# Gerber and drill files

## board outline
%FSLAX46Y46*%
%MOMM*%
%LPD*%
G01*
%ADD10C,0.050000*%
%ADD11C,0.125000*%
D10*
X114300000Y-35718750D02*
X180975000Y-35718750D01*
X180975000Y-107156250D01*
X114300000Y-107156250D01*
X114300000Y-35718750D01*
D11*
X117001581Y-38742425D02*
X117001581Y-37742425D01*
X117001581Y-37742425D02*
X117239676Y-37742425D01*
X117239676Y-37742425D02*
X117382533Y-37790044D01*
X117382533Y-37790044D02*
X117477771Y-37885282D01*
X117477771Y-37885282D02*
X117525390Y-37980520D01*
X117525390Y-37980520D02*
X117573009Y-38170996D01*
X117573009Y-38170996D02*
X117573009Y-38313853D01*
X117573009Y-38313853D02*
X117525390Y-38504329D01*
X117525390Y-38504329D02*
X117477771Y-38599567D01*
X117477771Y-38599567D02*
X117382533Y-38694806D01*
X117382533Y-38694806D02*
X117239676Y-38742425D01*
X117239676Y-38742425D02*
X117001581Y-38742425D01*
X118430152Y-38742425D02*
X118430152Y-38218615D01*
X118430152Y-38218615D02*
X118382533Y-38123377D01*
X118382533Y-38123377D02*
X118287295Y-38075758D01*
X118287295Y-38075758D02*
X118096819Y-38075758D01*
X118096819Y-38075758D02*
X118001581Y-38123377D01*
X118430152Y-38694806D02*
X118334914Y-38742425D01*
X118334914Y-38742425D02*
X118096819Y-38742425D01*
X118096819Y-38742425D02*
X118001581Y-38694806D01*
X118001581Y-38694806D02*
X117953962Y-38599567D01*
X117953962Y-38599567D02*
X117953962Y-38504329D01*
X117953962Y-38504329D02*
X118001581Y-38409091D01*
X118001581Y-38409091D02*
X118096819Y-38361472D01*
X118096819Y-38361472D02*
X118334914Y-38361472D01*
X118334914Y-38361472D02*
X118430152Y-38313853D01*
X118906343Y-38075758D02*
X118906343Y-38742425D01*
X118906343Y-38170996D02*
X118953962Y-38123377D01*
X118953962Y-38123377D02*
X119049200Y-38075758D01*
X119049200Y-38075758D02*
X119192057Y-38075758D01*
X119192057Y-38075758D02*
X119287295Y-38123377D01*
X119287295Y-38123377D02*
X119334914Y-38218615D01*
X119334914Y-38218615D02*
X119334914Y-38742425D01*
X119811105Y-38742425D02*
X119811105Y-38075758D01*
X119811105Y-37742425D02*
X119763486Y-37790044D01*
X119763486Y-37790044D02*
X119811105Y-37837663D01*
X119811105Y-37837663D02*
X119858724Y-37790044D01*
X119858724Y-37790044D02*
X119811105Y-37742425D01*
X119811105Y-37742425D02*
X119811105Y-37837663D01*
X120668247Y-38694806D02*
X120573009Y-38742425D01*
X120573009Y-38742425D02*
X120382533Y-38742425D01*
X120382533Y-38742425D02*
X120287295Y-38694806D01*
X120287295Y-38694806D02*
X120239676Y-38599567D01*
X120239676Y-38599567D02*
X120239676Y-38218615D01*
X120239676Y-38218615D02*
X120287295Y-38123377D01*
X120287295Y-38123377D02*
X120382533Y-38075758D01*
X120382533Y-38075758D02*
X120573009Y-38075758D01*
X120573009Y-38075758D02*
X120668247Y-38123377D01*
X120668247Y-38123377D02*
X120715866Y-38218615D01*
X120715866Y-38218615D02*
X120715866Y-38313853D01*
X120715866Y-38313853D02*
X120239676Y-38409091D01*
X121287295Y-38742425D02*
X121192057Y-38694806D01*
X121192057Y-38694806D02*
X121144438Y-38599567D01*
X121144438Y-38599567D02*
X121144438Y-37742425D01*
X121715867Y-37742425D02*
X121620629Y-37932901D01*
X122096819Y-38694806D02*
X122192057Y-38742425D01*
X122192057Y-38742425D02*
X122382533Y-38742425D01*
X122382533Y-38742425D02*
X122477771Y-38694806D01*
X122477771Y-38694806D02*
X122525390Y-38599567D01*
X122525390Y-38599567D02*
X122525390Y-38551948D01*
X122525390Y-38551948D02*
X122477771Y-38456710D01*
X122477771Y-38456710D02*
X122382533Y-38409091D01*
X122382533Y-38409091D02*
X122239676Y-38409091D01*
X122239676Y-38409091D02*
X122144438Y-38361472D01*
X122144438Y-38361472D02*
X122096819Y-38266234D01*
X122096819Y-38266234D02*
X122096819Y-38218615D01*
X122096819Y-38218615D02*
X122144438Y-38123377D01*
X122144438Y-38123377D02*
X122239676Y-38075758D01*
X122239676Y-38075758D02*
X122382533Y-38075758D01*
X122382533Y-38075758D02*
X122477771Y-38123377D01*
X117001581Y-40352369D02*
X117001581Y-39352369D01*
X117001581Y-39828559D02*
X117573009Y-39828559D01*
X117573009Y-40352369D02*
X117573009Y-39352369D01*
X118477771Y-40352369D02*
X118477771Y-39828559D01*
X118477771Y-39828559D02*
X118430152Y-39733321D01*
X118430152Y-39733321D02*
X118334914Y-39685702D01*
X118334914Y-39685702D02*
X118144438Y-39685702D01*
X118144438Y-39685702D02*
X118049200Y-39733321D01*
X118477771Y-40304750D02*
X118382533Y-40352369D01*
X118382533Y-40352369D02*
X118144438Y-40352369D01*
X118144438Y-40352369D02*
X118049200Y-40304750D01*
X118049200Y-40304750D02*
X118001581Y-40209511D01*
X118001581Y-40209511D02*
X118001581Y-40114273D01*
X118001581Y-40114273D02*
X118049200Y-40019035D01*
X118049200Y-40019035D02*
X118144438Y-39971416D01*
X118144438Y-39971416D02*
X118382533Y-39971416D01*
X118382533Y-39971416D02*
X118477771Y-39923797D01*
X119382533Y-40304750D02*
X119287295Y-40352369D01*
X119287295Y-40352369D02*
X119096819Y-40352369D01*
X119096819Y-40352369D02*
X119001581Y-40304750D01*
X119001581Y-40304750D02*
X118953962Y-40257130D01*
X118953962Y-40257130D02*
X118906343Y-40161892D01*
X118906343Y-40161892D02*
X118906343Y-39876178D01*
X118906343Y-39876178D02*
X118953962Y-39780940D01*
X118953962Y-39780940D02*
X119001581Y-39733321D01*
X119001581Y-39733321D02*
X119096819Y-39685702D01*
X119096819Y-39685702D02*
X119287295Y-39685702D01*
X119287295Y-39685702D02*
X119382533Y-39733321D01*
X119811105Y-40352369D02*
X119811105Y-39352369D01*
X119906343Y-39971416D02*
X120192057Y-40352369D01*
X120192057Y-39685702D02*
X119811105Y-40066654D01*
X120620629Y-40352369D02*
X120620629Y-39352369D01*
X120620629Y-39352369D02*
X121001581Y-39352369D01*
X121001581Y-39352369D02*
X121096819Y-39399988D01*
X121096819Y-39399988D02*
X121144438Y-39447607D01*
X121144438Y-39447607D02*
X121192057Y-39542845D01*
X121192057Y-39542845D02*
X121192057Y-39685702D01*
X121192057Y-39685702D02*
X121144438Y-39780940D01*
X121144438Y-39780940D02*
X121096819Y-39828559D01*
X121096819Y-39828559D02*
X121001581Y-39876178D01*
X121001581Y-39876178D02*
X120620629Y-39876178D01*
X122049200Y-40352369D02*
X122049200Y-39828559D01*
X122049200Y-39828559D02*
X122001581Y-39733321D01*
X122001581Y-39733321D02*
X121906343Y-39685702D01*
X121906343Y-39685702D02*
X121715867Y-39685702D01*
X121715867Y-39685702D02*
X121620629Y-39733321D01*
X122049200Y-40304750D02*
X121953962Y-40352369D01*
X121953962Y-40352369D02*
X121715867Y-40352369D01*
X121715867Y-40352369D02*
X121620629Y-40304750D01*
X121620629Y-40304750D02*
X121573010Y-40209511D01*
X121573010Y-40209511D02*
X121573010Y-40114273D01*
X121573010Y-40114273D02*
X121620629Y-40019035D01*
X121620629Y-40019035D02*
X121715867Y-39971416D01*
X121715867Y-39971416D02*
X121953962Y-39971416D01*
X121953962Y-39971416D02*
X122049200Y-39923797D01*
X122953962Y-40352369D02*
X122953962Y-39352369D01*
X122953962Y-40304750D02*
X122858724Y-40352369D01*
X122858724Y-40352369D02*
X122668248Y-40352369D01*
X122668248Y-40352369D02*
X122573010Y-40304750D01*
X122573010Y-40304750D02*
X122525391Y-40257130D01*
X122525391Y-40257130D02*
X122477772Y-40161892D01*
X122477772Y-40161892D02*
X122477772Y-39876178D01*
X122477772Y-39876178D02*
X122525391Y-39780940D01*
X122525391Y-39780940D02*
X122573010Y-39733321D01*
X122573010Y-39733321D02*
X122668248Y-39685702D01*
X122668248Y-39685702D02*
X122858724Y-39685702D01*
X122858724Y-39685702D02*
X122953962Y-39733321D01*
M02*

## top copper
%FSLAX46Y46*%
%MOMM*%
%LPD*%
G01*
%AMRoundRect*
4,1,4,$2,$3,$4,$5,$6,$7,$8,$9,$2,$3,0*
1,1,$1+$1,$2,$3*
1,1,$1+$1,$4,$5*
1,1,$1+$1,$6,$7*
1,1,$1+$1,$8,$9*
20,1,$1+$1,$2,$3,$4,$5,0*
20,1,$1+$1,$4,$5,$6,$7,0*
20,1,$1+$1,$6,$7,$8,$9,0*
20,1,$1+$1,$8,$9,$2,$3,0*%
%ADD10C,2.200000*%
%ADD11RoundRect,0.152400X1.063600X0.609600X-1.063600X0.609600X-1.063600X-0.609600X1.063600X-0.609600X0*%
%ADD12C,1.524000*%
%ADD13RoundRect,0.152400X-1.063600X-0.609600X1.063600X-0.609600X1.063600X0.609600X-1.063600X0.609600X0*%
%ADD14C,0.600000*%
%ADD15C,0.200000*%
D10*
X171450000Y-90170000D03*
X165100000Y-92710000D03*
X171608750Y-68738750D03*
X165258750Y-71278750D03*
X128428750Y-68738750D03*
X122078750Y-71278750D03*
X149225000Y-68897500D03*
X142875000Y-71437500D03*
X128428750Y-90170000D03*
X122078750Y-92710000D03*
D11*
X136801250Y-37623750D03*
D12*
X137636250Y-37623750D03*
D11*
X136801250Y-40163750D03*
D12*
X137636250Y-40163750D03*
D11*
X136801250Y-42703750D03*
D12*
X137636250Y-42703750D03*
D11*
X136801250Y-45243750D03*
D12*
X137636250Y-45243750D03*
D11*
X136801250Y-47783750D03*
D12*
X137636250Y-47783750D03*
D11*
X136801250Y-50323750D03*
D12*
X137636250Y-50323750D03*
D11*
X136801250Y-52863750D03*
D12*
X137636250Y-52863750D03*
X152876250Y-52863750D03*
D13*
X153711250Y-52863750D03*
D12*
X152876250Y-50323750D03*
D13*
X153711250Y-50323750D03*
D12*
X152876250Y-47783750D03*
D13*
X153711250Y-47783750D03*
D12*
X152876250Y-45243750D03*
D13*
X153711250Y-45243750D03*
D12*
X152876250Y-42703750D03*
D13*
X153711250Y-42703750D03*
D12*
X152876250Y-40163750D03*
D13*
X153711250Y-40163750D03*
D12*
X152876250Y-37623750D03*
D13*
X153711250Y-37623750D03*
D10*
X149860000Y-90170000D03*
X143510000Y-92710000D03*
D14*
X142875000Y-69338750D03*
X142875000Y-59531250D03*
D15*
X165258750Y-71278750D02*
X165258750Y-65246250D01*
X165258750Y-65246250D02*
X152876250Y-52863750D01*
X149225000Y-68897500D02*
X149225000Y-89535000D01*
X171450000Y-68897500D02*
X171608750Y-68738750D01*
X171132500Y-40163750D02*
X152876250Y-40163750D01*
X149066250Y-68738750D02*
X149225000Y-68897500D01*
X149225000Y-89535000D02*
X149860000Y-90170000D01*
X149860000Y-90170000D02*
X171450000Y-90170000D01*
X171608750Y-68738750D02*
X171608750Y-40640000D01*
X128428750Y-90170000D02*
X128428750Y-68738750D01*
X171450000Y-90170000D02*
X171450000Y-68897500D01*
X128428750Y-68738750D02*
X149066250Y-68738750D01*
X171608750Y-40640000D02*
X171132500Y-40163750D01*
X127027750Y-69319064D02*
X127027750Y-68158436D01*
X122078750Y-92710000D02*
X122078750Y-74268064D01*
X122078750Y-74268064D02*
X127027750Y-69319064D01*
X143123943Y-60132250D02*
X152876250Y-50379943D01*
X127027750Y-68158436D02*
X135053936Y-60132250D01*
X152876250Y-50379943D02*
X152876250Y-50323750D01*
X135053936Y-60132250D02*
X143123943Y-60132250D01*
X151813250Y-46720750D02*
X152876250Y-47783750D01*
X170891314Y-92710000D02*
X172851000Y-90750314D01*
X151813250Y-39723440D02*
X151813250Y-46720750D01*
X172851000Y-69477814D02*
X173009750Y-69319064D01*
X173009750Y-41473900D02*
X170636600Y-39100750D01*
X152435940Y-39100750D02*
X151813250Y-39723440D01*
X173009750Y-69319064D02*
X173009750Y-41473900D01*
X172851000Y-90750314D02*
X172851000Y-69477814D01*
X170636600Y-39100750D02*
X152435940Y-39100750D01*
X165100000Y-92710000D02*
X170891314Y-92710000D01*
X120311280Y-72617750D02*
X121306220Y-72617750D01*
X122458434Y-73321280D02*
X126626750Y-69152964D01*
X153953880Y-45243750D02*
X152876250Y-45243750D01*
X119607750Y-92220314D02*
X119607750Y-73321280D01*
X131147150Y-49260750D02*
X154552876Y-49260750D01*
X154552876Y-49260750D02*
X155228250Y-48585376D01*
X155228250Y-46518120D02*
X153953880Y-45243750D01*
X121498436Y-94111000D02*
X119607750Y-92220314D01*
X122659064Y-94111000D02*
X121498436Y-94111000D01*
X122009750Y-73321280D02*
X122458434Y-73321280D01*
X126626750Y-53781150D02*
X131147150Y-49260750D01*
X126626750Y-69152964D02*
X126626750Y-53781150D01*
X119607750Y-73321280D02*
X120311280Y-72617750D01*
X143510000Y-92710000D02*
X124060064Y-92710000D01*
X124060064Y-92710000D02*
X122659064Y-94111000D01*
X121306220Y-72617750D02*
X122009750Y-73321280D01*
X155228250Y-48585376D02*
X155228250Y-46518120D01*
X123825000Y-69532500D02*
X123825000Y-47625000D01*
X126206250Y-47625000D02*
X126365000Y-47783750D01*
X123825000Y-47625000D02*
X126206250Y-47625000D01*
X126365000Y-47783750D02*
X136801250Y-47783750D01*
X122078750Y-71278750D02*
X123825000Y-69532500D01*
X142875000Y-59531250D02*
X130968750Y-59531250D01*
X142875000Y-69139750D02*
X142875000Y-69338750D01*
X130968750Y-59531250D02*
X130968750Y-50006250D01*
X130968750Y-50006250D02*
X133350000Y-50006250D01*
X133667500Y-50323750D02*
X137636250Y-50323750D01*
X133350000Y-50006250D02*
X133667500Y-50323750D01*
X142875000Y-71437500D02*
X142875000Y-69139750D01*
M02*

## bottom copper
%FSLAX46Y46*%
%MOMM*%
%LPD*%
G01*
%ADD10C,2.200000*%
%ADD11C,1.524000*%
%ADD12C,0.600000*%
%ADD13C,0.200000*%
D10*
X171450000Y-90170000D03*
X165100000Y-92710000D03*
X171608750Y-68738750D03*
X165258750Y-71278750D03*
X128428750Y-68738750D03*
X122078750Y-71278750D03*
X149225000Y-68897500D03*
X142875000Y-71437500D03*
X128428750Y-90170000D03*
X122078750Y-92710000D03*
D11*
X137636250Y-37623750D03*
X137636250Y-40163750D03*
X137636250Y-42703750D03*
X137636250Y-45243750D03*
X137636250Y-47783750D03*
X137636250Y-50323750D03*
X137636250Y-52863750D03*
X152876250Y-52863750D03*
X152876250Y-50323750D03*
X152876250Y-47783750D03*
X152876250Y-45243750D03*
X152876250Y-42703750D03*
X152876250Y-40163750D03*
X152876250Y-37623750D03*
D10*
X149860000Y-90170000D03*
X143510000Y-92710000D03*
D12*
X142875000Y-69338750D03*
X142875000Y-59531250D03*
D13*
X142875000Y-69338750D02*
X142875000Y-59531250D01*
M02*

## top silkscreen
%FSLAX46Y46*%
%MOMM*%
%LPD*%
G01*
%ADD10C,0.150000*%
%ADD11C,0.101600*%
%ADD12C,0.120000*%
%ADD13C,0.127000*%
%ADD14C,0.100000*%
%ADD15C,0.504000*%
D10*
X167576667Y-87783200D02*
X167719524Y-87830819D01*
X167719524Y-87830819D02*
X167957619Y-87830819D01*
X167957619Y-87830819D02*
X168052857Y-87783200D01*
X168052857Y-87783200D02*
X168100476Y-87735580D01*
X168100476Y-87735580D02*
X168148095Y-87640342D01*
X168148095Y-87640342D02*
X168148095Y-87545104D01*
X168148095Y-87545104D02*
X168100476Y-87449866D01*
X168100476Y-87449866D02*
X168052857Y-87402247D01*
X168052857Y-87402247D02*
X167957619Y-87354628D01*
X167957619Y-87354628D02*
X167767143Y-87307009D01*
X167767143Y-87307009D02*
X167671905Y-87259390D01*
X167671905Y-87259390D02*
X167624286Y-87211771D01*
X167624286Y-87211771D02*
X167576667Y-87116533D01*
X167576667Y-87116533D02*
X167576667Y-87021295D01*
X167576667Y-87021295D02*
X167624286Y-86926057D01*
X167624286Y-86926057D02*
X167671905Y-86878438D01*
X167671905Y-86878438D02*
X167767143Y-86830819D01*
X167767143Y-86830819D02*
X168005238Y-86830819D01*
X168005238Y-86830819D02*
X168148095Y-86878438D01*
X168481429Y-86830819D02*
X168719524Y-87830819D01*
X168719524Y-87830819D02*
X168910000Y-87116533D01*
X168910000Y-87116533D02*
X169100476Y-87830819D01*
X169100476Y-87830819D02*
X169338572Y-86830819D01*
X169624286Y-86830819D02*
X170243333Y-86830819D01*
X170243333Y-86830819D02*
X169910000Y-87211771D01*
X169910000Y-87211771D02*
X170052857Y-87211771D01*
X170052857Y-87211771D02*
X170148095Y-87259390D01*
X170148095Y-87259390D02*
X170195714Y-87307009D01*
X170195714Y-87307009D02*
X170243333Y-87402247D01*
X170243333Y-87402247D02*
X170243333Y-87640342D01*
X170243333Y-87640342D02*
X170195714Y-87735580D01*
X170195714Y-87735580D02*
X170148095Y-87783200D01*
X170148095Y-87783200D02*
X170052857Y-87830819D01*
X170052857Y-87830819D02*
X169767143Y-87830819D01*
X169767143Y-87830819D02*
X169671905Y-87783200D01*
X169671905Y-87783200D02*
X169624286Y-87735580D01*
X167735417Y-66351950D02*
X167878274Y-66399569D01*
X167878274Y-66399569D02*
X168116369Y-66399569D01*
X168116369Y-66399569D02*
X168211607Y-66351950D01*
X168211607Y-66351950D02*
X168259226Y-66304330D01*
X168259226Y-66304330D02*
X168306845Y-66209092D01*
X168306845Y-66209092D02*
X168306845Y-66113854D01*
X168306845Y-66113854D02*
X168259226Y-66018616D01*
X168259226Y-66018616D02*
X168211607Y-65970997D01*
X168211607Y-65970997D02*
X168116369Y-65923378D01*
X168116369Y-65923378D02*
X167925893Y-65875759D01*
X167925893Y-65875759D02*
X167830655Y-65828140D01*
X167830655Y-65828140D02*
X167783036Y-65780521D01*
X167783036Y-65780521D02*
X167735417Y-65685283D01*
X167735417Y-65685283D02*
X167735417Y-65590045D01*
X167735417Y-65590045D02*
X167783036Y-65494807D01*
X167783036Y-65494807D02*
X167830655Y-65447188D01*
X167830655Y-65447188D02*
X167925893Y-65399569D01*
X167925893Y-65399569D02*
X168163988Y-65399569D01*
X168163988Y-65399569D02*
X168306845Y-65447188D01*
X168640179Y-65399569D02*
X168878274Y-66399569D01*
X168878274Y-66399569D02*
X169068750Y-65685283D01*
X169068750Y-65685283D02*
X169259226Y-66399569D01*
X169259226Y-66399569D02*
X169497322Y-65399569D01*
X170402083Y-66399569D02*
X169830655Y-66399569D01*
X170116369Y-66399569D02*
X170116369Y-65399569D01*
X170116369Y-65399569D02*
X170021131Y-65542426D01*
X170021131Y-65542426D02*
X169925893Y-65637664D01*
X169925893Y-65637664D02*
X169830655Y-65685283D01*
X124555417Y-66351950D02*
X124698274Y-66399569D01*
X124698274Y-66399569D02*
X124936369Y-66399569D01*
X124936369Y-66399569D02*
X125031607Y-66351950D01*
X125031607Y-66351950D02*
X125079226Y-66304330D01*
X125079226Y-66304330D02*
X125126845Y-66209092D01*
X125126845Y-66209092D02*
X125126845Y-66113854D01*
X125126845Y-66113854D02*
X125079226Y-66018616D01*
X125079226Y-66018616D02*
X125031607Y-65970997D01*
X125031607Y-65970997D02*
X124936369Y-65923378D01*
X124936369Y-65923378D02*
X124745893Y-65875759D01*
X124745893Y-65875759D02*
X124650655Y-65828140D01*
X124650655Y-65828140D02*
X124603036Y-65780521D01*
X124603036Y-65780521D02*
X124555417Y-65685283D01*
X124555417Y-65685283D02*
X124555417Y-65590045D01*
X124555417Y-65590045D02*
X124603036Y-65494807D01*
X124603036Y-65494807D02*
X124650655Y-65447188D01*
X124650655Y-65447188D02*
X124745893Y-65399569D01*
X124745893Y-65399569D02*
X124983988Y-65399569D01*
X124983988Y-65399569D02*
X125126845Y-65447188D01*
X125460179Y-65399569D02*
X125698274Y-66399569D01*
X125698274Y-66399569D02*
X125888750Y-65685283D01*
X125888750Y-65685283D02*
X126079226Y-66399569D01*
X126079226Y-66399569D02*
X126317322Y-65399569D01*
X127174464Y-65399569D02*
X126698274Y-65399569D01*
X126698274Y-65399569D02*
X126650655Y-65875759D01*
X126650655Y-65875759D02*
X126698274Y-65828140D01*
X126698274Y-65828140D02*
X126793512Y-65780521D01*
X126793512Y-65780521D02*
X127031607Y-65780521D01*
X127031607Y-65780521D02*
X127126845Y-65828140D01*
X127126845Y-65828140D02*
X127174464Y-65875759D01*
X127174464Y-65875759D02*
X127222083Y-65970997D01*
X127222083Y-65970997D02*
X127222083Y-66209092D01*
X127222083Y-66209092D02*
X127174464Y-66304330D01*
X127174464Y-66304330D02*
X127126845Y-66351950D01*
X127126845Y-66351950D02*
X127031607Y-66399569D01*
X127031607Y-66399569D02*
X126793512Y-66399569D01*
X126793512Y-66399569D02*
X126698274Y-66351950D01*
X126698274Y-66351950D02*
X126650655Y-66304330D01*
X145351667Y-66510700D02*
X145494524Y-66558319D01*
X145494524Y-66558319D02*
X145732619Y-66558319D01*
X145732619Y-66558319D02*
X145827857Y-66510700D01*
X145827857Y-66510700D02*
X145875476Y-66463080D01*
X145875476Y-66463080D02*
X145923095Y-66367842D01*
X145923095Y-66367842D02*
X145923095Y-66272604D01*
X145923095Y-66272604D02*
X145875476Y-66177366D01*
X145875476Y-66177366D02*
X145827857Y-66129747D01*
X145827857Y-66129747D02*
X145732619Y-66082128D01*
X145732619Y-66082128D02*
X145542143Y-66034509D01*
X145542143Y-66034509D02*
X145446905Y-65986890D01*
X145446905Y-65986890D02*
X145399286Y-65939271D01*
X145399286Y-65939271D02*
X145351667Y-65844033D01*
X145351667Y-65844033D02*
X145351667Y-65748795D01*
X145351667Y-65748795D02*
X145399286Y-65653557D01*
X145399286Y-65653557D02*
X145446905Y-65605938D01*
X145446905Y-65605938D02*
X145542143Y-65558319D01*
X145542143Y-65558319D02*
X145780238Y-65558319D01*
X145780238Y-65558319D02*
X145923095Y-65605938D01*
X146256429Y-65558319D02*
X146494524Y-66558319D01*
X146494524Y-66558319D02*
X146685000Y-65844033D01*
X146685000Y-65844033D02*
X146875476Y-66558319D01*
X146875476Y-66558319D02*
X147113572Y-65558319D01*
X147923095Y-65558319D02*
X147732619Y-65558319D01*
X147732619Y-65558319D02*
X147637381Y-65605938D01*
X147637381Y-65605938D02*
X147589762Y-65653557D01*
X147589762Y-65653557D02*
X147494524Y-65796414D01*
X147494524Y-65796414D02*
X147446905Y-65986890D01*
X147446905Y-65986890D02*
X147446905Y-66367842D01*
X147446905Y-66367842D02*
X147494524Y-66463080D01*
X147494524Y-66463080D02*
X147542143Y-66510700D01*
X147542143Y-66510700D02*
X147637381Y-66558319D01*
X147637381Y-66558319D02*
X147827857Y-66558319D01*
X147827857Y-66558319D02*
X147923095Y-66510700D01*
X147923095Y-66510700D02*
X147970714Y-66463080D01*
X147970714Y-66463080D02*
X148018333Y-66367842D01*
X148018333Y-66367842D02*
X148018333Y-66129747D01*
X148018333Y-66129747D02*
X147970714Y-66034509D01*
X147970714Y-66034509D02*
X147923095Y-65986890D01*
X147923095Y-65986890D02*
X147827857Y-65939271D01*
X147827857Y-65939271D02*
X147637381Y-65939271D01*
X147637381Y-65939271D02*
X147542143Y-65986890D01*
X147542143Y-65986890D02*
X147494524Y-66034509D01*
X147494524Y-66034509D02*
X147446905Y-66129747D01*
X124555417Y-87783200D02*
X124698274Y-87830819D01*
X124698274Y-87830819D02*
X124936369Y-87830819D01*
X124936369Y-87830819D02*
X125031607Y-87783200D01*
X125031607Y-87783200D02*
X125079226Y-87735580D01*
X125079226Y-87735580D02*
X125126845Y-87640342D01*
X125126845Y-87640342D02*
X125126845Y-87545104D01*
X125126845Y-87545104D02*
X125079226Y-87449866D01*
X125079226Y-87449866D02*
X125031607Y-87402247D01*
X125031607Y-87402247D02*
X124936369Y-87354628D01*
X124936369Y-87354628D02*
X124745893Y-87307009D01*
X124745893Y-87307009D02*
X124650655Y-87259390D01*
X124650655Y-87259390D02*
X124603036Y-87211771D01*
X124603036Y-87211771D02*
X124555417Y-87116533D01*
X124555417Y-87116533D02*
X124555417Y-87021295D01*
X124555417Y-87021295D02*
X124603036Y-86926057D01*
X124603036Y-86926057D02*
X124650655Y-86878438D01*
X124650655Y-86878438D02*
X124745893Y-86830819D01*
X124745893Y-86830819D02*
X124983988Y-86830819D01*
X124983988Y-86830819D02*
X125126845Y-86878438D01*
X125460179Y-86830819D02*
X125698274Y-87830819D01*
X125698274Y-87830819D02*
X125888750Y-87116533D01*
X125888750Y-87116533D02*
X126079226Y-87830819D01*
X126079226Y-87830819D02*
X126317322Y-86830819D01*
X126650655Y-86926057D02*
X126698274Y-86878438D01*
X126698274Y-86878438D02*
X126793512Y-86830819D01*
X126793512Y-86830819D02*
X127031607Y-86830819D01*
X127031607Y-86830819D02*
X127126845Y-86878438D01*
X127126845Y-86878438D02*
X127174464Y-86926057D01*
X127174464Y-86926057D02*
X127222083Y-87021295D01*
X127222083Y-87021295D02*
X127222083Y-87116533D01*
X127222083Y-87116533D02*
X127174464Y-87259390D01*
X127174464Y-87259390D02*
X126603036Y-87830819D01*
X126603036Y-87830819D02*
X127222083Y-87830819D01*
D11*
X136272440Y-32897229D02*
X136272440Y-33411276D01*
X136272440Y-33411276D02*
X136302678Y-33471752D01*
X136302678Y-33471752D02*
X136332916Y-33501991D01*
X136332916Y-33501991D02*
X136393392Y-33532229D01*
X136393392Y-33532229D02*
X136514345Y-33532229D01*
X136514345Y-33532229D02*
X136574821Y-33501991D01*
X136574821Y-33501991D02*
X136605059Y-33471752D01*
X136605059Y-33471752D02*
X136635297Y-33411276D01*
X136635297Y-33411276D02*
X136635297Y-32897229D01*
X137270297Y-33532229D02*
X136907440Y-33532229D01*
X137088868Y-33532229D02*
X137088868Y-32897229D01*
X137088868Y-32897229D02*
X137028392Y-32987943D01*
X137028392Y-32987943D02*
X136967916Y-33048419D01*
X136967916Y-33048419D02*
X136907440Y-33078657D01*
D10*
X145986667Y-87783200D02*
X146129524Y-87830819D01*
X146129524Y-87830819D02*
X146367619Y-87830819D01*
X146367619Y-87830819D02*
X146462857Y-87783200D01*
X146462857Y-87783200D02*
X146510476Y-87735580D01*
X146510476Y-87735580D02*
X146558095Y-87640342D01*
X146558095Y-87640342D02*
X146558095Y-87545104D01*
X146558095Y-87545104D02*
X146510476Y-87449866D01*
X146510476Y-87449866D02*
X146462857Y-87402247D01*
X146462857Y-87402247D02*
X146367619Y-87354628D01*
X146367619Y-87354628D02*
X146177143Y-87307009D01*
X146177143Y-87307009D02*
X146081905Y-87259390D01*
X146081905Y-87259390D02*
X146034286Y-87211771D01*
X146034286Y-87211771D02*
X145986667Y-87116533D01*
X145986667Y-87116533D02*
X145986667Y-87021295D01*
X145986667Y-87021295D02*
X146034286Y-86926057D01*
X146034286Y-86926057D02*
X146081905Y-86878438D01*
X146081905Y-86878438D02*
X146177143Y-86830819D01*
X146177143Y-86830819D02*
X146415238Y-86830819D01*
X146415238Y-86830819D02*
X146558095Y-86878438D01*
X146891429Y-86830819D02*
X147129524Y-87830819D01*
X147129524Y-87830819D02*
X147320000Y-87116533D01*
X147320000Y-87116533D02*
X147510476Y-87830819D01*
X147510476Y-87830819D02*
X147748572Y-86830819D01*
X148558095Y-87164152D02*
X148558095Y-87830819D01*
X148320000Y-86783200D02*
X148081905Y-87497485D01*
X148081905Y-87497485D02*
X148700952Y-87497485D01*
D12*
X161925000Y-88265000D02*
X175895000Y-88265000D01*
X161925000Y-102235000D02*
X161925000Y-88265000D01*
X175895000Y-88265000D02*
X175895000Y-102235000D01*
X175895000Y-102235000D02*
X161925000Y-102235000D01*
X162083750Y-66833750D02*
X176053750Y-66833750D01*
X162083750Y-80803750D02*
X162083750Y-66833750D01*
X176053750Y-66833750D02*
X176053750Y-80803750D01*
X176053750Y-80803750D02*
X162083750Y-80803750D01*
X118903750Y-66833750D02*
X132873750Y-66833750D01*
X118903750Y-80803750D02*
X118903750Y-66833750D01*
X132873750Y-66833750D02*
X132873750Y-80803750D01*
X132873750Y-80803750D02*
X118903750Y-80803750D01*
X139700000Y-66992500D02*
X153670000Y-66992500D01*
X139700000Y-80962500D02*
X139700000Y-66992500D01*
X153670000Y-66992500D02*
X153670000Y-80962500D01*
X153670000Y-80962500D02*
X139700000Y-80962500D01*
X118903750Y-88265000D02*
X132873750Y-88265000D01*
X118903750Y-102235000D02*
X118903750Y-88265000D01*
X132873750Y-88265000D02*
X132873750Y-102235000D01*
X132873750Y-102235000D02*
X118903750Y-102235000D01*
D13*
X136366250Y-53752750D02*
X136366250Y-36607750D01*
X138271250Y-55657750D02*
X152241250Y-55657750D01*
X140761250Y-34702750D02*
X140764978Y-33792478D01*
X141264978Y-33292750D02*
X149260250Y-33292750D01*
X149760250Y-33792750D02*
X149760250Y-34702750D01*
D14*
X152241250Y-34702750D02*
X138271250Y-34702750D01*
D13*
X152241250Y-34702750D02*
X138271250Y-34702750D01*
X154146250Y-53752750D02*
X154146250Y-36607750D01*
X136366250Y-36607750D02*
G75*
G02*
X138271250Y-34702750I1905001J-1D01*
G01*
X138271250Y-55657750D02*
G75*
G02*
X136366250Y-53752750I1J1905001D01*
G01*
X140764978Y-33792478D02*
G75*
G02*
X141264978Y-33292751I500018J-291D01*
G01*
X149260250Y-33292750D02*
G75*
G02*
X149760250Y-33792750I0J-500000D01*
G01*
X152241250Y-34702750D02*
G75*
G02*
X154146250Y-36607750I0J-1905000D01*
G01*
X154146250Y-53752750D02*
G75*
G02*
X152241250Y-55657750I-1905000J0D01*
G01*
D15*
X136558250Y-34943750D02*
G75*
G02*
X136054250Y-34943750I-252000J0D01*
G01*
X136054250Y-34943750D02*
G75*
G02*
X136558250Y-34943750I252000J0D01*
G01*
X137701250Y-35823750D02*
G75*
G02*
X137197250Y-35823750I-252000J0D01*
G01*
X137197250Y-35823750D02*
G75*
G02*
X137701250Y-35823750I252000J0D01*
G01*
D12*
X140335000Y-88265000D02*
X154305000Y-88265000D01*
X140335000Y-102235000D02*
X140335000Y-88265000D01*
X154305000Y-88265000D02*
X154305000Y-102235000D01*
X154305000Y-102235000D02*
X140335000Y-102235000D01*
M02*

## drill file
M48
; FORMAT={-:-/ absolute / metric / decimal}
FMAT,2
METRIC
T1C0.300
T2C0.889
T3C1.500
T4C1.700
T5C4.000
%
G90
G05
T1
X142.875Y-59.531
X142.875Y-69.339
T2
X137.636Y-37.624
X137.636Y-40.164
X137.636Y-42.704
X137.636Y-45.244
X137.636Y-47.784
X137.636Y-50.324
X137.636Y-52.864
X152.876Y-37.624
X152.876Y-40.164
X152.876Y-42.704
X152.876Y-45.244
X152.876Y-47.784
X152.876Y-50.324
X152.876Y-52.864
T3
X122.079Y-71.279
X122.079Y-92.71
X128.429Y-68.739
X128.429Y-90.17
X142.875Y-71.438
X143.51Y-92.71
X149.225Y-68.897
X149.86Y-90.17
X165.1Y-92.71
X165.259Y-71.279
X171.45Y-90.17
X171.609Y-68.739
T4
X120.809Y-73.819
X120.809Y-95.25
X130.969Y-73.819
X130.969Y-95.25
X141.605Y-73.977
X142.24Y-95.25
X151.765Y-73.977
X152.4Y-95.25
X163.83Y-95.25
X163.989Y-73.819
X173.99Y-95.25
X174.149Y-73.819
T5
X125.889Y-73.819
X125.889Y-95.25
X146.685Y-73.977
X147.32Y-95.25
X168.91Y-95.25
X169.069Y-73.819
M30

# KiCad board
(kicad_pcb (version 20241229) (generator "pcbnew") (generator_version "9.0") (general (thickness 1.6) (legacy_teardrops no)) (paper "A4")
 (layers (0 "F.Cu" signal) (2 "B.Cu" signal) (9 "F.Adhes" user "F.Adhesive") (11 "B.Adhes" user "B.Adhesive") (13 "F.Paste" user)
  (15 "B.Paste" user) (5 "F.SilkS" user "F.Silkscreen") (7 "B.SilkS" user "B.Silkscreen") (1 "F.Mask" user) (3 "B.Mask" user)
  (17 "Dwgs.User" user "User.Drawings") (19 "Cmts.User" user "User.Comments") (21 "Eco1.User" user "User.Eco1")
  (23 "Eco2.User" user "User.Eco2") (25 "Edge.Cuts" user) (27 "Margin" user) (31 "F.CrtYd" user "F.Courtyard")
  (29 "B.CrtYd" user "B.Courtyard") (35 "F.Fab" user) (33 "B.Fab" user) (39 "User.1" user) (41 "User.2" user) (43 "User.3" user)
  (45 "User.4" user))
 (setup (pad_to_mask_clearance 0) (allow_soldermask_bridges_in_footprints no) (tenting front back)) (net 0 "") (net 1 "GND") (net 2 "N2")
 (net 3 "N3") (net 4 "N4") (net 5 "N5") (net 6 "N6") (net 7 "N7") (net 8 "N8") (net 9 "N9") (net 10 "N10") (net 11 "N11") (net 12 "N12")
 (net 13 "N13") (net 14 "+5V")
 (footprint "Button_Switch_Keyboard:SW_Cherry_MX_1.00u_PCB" (layer "F.Cu") (at 171.45 90.17)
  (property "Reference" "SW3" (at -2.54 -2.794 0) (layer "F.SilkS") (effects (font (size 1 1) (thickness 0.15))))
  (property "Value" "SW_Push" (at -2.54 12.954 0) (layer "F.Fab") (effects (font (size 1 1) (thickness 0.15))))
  (fp_line (start -9.525 -1.905) (end 4.445 -1.905) (stroke (width 0.12) (type solid)) (layer "F.SilkS"))
  (fp_line (start -9.525 12.065) (end -9.525 -1.905) (stroke (width 0.12) (type solid)) (layer "F.SilkS"))
  (fp_line (start 4.445 -1.905) (end 4.445 12.065) (stroke (width 0.12) (type solid)) (layer "F.SilkS"))
  (fp_line (start 4.445 12.065) (end -9.525 12.065) (stroke (width 0.12) (type solid)) (layer "F.SilkS"))
  (pad "" np_thru_hole circle (at -7.62 5.08) (size 1.7 1.7) (drill 1.7) (layers "*.Cu" "*.Mask"))
  (pad "" np_thru_hole circle (at -2.54 5.08) (size 4 4) (drill 4) (layers "*.Cu" "*.Mask"))
  (pad "" np_thru_hole circle (at 2.54 5.08) (size 1.7 1.7) (drill 1.7) (layers "*.Cu" "*.Mask"))
  (pad "1" thru_hole circle (at 0 0) (size 2.2 2.2) (drill 1.5) (layers "*.Cu" "*.Mask") (remove_unused_layers no) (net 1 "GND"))
  (pad "2" thru_hole circle (at -6.35 2.54) (size 2.2 2.2) (drill 1.5) (layers "*.Cu" "*.Mask") (remove_unused_layers no) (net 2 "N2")))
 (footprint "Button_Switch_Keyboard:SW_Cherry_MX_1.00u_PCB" (layer "F.Cu") (at 171.60875 68.73875)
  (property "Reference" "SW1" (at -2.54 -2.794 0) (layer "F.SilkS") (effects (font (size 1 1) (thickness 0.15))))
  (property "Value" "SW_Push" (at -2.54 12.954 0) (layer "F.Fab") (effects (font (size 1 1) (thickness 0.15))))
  (fp_line (start -9.525 -1.905) (end 4.445 -1.905) (stroke (width 0.12) (type solid)) (layer "F.SilkS"))
  (fp_line (start -9.525 12.065) (end -9.525 -1.905) (stroke (width 0.12) (type solid)) (layer "F.SilkS"))
  (fp_line (start 4.445 -1.905) (end 4.445 12.065) (stroke (width 0.12) (type solid)) (layer "F.SilkS"))
  (fp_line (start 4.445 12.065) (end -9.525 12.065) (stroke (width 0.12) (type solid)) (layer "F.SilkS"))
  (pad "" np_thru_hole circle (at -7.62 5.08) (size 1.7 1.7) (drill 1.7) (layers "*.Cu" "*.Mask"))
  (pad "" np_thru_hole circle (at -2.54 5.08) (size 4 4) (drill 4) (layers "*.Cu" "*.Mask"))
  (pad "" np_thru_hole circle (at 2.54 5.08) (size 1.7 1.7) (drill 1.7) (layers "*.Cu" "*.Mask"))
  (pad "1" thru_hole circle (at 0 0) (size 2.2 2.2) (drill 1.5) (layers "*.Cu" "*.Mask") (remove_unused_layers no) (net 1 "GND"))
  (pad "2" thru_hole circle (at -6.35 2.54) (size 2.2 2.2) (drill 1.5) (layers "*.Cu" "*.Mask") (remove_unused_layers no) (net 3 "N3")))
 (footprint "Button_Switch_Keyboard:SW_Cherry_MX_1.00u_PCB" (layer "F.Cu") (at 128.42875 68.73875)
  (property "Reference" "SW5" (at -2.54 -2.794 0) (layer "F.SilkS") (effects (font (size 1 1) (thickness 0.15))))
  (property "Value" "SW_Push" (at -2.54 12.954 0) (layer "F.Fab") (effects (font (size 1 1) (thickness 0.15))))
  (fp_line (start -9.525 -1.905) (end 4.445 -1.905) (stroke (width 0.12) (type solid)) (layer "F.SilkS"))
  (fp_line (start -9.525 12.065) (end -9.525 -1.905) (stroke (width 0.12) (type solid)) (layer "F.SilkS"))
  (fp_line (start 4.445 -1.905) (end 4.445 12.065) (stroke (width 0.12) (type solid)) (layer "F.SilkS"))
  (fp_line (start 4.445 12.065) (end -9.525 12.065) (stroke (width 0.12) (type solid)) (layer "F.SilkS"))
  (pad "" np_thru_hole circle (at -7.62 5.08) (size 1.7 1.7) (drill 1.7) (layers "*.Cu" "*.Mask"))
  (pad "" np_thru_hole circle (at -2.54 5.08) (size 4 4) (drill 4) (layers "*.Cu" "*.Mask"))
  (pad "" np_thru_hole circle (at 2.54 5.08) (size 1.7 1.7) (drill 1.7) (layers "*.Cu" "*.Mask"))
  (pad "1" thru_hole circle (at 0 0) (size 2.2 2.2) (drill 1.5) (layers "*.Cu" "*.Mask") (remove_unused_layers no) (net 1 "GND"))
  (pad "2" thru_hole circle (at -6.35 2.54) (size 2.2 2.2) (drill 1.5) (layers "*.Cu" "*.Mask") (remove_unused_layers no) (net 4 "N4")))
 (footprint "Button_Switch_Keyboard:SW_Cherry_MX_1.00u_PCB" (layer "F.Cu") (at 149.225 68.8975)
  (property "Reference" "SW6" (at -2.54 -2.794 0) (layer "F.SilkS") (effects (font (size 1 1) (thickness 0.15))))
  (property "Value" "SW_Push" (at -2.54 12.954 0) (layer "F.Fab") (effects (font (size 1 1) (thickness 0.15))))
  (fp_line (start -9.525 -1.905) (end 4.445 -1.905) (stroke (width 0.12) (type solid)) (layer "F.SilkS"))
  (fp_line (start -9.525 12.065) (end -9.525 -1.905) (stroke (width 0.12) (type solid)) (layer "F.SilkS"))
  (fp_line (start 4.445 -1.905) (end 4.445 12.065) (stroke (width 0.12) (type solid)) (layer "F.SilkS"))
  (fp_line (start 4.445 12.065) (end -9.525 12.065) (stroke (width 0.12) (type solid)) (layer "F.SilkS"))
  (pad "" np_thru_hole circle (at -7.62 5.08) (size 1.7 1.7) (drill 1.7) (layers "*.Cu" "*.Mask"))
  (pad "" np_thru_hole circle (at -2.54 5.08) (size 4 4) (drill 4) (layers "*.Cu" "*.Mask"))
  (pad "" np_thru_hole circle (at 2.54 5.08) (size 1.7 1.7) (drill 1.7) (layers "*.Cu" "*.Mask"))
  (pad "1" thru_hole circle (at 0 0) (size 2.2 2.2) (drill 1.5) (layers "*.Cu" "*.Mask") (remove_unused_layers no) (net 1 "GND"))
  (pad "2" thru_hole circle (at -6.35 2.54) (size 2.2 2.2) (drill 1.5) (layers "*.Cu" "*.Mask") (remove_unused_layers no) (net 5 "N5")))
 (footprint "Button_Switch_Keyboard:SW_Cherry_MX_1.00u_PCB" (layer "F.Cu") (at 128.42875 90.17)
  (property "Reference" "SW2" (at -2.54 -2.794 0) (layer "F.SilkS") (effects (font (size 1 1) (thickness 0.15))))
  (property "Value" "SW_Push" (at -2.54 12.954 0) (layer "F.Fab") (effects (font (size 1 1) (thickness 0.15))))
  (fp_line (start -9.525 -1.905) (end 4.445 -1.905) (stroke (width 0.12) (type solid)) (layer "F.SilkS"))
  (fp_line (start -9.525 12.065) (end -9.525 -1.905) (stroke (width 0.12) (type solid)) (layer "F.SilkS"))
  (fp_line (start 4.445 -1.905) (end 4.445 12.065) (stroke (width 0.12) (type solid)) (layer "F.SilkS"))
  (fp_line (start 4.445 12.065) (end -9.525 12.065) (stroke (width 0.12) (type solid)) (layer "F.SilkS"))
  (pad "" np_thru_hole circle (at -7.62 5.08) (size 1.7 1.7) (drill 1.7) (layers "*.Cu" "*.Mask"))
  (pad "" np_thru_hole circle (at -2.54 5.08) (size 4 4) (drill 4) (layers "*.Cu" "*.Mask"))
  (pad "" np_thru_hole circle (at 2.54 5.08) (size 1.7 1.7) (drill 1.7) (layers "*.Cu" "*.Mask"))
  (pad "1" thru_hole circle (at 0 0) (size 2.2 2.2) (drill 1.5) (layers "*.Cu" "*.Mask") (remove_unused_layers no) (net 1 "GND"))
  (pad "2" thru_hole circle (at -6.35 2.54) (size 2.2 2.2) (drill 1.5) (layers "*.Cu" "*.Mask") (remove_unused_layers no) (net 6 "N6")))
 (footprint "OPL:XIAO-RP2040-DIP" (layer "F.Cu") (at 145.25625 45.24375)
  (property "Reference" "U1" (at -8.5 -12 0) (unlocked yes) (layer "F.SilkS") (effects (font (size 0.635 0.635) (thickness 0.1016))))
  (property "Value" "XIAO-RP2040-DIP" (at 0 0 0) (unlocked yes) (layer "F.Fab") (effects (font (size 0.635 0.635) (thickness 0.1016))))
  (fp_line (start -8.89 8.509) (end -8.89 -8.636) (stroke (width 0.127) (type solid)) (layer "F.SilkS"))
  (fp_line (start -6.985 10.414) (end 6.985 10.414) (stroke (width 0.127) (type solid)) (layer "F.SilkS"))
  (fp_line (start -4.495 -10.541) (end -4.491272 -11.451272) (stroke (width 0.127) (type solid)) (layer "F.SilkS"))
  (fp_line (start -3.991272 -11.951) (end 4.004 -11.951) (stroke (width 0.127) (type solid)) (layer "F.SilkS"))
  (fp_line (start 4.504 -11.451) (end 4.504 -10.541) (stroke (width 0.127) (type solid)) (layer "F.SilkS"))
  (fp_line (start 6.985 -10.541) (end -6.985 -10.541) (stroke (width 0.1) (type solid)) (layer "F.SilkS"))
  (fp_line (start 6.985 -10.541) (end -6.985 -10.541) (stroke (width 0.127) (type solid)) (layer "F.SilkS"))
  (fp_line (start 8.89 8.509) (end 8.89 -8.636) (stroke (width 0.127) (type solid)) (layer "F.SilkS"))
  (fp_arc (start -8.89 -8.636) (mid -8.332038 -9.983038) (end -6.985 -10.541) (stroke (width 0.127) (type solid)) (layer "F.SilkS"))
  (fp_arc (start -6.985 10.414) (mid -8.332038 9.856038) (end -8.89 8.509) (stroke (width 0.127) (type solid)) (layer "F.SilkS"))
  (fp_arc (start -4.491272 -11.451272) (mid -4.344728 -11.80464) (end -3.991272 -11.951) (stroke (width 0.127) (type default))
   (layer "F.SilkS"))
  (fp_arc (start 4.004 -11.951) (mid 4.357553 -11.804553) (end 4.504 -11.451) (stroke (width 0.127) (type default)) (layer "F.SilkS"))
  (fp_arc (start 6.985 -10.541) (mid 8.332038 -9.983038) (end 8.89 -8.636) (stroke (width 0.127) (type solid)) (layer "F.SilkS"))
  (fp_arc (start 8.89 8.509) (mid 8.332038 9.856038) (end 6.985 10.414) (stroke (width 0.127) (type solid)) (layer "F.SilkS"))
  (fp_circle (center -8.95 -10.3) (end -8.95 -10.554) (stroke (width 0.5) (type solid)) (fill yes) (layer "F.SilkS"))
  (fp_circle (center -7.807 -9.42) (end -7.807 -9.674) (stroke (width 0.5) (type solid)) (fill yes) (layer "F.SilkS"))
  (pad "1" smd roundrect (at -8.455 -7.62 180) (size 2.432 1.524) (layers "F.Cu" "F.Mask") (roundrect_rratio 0.1) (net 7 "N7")
   (thermal_bridge_angle 45))
  (pad "1" thru_hole circle (at -7.62 -7.62 180) (size 1.524 1.524) (drill 0.889) (layers "*.Cu" "*.Mask") (remove_unused_layers no)
   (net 7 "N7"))
  (pad "2" smd roundrect (at -8.455 -5.08 180) (size 2.432 1.524) (layers "F.Cu" "F.Mask") (roundrect_rratio 0.1) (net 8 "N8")
   (thermal_bridge_angle 45))
  (pad "2" thru_hole circle (at -7.62 -5.08 180) (size 1.524 1.524) (drill 0.889) (layers "*.Cu" "*.Mask") (remove_unused_layers no)
   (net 8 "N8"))
  (pad "3" smd roundrect (at -8.455 -2.54 180) (size 2.432 1.524) (layers "F.Cu" "F.Mask") (roundrect_rratio 0.1) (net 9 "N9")
   (thermal_bridge_angle 45))
  (pad "3" thru_hole circle (at -7.62 -2.54 180) (size 1.524 1.524) (drill 0.889) (layers "*.Cu" "*.Mask") (remove_unused_layers no)
   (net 9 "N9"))
  (pad "4" smd roundrect (at -8.455 0 180) (size 2.432 1.524) (layers "F.Cu" "F.Mask") (roundrect_rratio 0.1) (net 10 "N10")
   (thermal_bridge_angle 45))
  (pad "4" thru_hole circle (at -7.62 0 180) (size 1.524 1.524) (drill 0.889) (layers "*.Cu" "*.Mask") (remove_unused_layers no)
   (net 10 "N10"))
  (pad "5" smd roundrect (at -8.455 2.54 180) (size 2.432 1.524) (layers "F.Cu" "F.Mask") (roundrect_rratio 0.1) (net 4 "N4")
   (thermal_bridge_angle 45))
  (pad "5" thru_hole circle (at -7.62 2.54 180) (size 1.524 1.524) (drill 0.889) (layers "*.Cu" "*.Mask") (remove_unused_layers no)
   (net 4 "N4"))
  (pad "6" smd roundrect (at -8.455 5.08 180) (size 2.432 1.524) (layers "F.Cu" "F.Mask") (roundrect_rratio 0.1) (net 5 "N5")
   (thermal_bridge_angle 45))
  (pad "6" thru_hole circle (at -7.62 5.08 180) (size 1.524 1.524) (drill 0.889) (layers "*.Cu" "*.Mask") (remove_unused_layers no)
   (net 5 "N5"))
  (pad "7" smd roundrect (at -8.455 7.62 180) (size 2.432 1.524) (layers "F.Cu" "F.Mask") (roundrect_rratio 0.1) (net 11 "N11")
   (thermal_bridge_angle 45))
  (pad "7" thru_hole circle (at -7.62 7.62 180) (size 1.524 1.524) (drill 0.889) (layers "*.Cu" "*.Mask") (remove_unused_layers no)
   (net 11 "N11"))
  (pad "8" thru_hole circle (at 7.62 7.62) (size 1.524 1.524) (drill 0.889) (layers "*.Cu" "*.Mask") (remove_unused_layers no) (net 3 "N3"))
  (pad "8" smd roundrect (at 8.455 7.62) (size 2.432 1.524) (layers "F.Cu" "F.Mask") (roundrect_rratio 0.1) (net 3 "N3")
   (thermal_bridge_angle 45))
  (pad "9" thru_hole circle (at 7.62 5.08) (size 1.524 1.524) (drill 0.889) (layers "*.Cu" "*.Mask") (remove_unused_layers no) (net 6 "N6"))
  (pad "9" smd roundrect (at 8.455 5.08) (size 2.432 1.524) (layers "F.Cu" "F.Mask") (roundrect_rratio 0.1) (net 6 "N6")
   (thermal_bridge_angle 45))
  (pad "10" thru_hole circle (at 7.62 2.54) (size 1.524 1.524) (drill 0.889) (layers "*.Cu" "*.Mask") (remove_unused_layers no) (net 2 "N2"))
  (pad "10" smd roundrect (at 8.455 2.54) (size 2.432 1.524) (layers "F.Cu" "F.Mask") (roundrect_rratio 0.1) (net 2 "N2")
   (thermal_bridge_angle 45))
  (pad "11" thru_hole circle (at 7.62 0) (size 1.524 1.524) (drill 0.889) (layers "*.Cu" "*.Mask") (remove_unused_layers no) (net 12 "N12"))
  (pad "11" smd roundrect (at 8.455 0) (size 2.432 1.524) (layers "F.Cu" "F.Mask") (roundrect_rratio 0.1) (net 12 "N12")
   (thermal_bridge_angle 45))
  (pad "12" thru_hole circle (at 7.62 -2.54) (size 1.524 1.524) (drill 0.889) (layers "*.Cu" "*.Mask") (remove_unused_layers no)
   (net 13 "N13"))
  (pad "12" smd roundrect (at 8.455 -2.54) (size 2.432 1.524) (layers "F.Cu" "F.Mask") (roundrect_rratio 0.1) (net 13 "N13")
   (thermal_bridge_angle 45))
  (pad "13" thru_hole circle (at 7.62 -5.08) (size 1.524 1.524) (drill 0.889) (layers "*.Cu" "*.Mask") (remove_unused_layers no)
   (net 1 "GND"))
  (pad "13" smd roundrect (at 8.455 -5.08) (size 2.432 1.524) (layers "F.Cu" "F.Mask") (roundrect_rratio 0.1) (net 1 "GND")
   (thermal_bridge_angle 45))
  (pad "14" thru_hole circle (at 7.62 -7.62) (size 1.524 1.524) (drill 0.889) (layers "*.Cu" "*.Mask") (remove_unused_layers no)
   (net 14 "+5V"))
  (pad "14" smd roundrect (at 8.455 -7.62) (size 2.432 1.524) (layers "F.Cu" "F.Mask") (roundrect_rratio 0.1) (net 14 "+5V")
   (thermal_bridge_angle 45)))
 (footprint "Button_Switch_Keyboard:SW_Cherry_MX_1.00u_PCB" (layer "F.Cu") (at 149.86 90.17)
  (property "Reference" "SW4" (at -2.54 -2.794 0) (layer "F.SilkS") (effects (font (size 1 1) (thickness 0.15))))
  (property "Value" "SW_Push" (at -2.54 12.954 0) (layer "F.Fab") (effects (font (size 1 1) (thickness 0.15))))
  (fp_line (start -9.525 -1.905) (end 4.445 -1.905) (stroke (width 0.12) (type solid)) (layer "F.SilkS"))
  (fp_line (start -9.525 12.065) (end -9.525 -1.905) (stroke (width 0.12) (type solid)) (layer "F.SilkS"))
  (fp_line (start 4.445 -1.905) (end 4.445 12.065) (stroke (width 0.12) (type solid)) (layer "F.SilkS"))
  (fp_line (start 4.445 12.065) (end -9.525 12.065) (stroke (width 0.12) (type solid)) (layer "F.SilkS"))
  (pad "" np_thru_hole circle (at -7.62 5.08) (size 1.7 1.7) (drill 1.7) (layers "*.Cu" "*.Mask"))
  (pad "" np_thru_hole circle (at -2.54 5.08) (size 4 4) (drill 4) (layers "*.Cu" "*.Mask"))
  (pad "" np_thru_hole circle (at 2.54 5.08) (size 1.7 1.7) (drill 1.7) (layers "*.Cu" "*.Mask"))
  (pad "1" thru_hole circle (at 0 0) (size 2.2 2.2) (drill 1.5) (layers "*.Cu" "*.Mask") (remove_unused_layers no) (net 1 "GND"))
  (pad "2" thru_hole circle (at -6.35 2.54) (size 2.2 2.2) (drill 1.5) (layers "*.Cu" "*.Mask") (remove_unused_layers no) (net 12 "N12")))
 (gr_rect (start 114.3 35.71875) (end 180.975 107.15625) (stroke (width 0.05) (type default)) (fill no) (layer "Edge.Cuts"))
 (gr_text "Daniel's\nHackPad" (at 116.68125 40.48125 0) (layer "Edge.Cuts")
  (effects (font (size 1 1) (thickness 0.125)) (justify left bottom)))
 (segment (start 165.25875 71.27875) (end 165.25875 65.24625) (width 0.2) (layer "F.Cu") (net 3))
 (segment (start 165.25875 65.24625) (end 152.87625 52.86375) (width 0.2) (layer "F.Cu") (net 3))
 (segment (start 149.225 68.8975) (end 149.225 89.535) (width 0.2) (layer "F.Cu") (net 1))
 (segment (start 171.45 68.8975) (end 171.60875 68.73875) (width 0.2) (layer "F.Cu") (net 1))
 (segment (start 171.1325 40.16375) (end 152.87625 40.16375) (width 0.2) (layer "F.Cu") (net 1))
 (segment (start 149.06625 68.73875) (end 149.225 68.8975) (width 0.2) (layer "F.Cu") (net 1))
 (segment (start 149.225 89.535) (end 149.86 90.17) (width 0.2) (layer "F.Cu") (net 1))
 (segment (start 149.86 90.17) (end 171.45 90.17) (width 0.2) (layer "F.Cu") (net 1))
 (segment (start 171.60875 68.73875) (end 171.60875 40.64) (width 0.2) (layer "F.Cu") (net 1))
 (segment (start 128.42875 90.17) (end 128.42875 68.73875) (width 0.2) (layer "F.Cu") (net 1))
 (segment (start 171.45 90.17) (end 171.45 68.8975) (width 0.2) (layer "F.Cu") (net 1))
 (segment (start 128.42875 68.73875) (end 149.06625 68.73875) (width 0.2) (layer "F.Cu") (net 1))
 (segment (start 171.60875 40.64) (end 171.1325 40.16375) (width 0.2) (layer "F.Cu") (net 1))
 (segment (start 127.02775 69.319064) (end 127.02775 68.158436) (width 0.2) (layer "F.Cu") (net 6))
 (segment (start 122.07875 92.71) (end 122.07875 74.268064) (width 0.2) (layer "F.Cu") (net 6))
 (segment (start 122.07875 74.268064) (end 127.02775 69.319064) (width 0.2) (layer "F.Cu") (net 6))
 (segment (start 143.123943 60.13225) (end 152.87625 50.379943) (width 0.2) (layer "F.Cu") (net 6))
 (segment (start 127.02775 68.158436) (end 135.053936 60.13225) (width 0.2) (layer "F.Cu") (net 6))
 (segment (start 152.87625 50.379943) (end 152.87625 50.32375) (width 0.2) (layer "F.Cu") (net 6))
 (segment (start 135.053936 60.13225) (end 143.123943 60.13225) (width 0.2) (layer "F.Cu") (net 6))
 (segment (start 151.81325 46.72075) (end 152.87625 47.78375) (width 0.2) (layer "F.Cu") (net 2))
 (segment (start 170.891314 92.71) (end 172.851 90.750314) (width 0.2) (layer "F.Cu") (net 2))
 (segment (start 151.81325 39.72344) (end 151.81325 46.72075) (width 0.2) (layer "F.Cu") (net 2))
 (segment (start 172.851 69.477814) (end 173.00975 69.319064) (width 0.2) (layer "F.Cu") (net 2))
 (segment (start 173.00975 41.4739) (end 170.6366 39.10075) (width 0.2) (layer "F.Cu") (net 2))
 (segment (start 152.43594 39.10075) (end 151.81325 39.72344) (width 0.2) (layer "F.Cu") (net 2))
 (segment (start 173.00975 69.319064) (end 173.00975 41.4739) (width 0.2) (layer "F.Cu") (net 2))
 (segment (start 172.851 90.750314) (end 172.851 69.477814) (width 0.2) (layer "F.Cu") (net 2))
 (segment (start 170.6366 39.10075) (end 152.43594 39.10075) (width 0.2) (layer "F.Cu") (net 2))
 (segment (start 165.1 92.71) (end 170.891314 92.71) (width 0.2) (layer "F.Cu") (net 2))
 (segment (start 120.31128 72.61775) (end 121.30622 72.61775) (width 0.2) (layer "F.Cu") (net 12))
 (segment (start 122.458434 73.32128) (end 126.62675 69.152964) (width 0.2) (layer "F.Cu") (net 12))
 (segment (start 153.95388 45.24375) (end 152.87625 45.24375) (width 0.2) (layer "F.Cu") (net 12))
 (segment (start 119.60775 92.220314) (end 119.60775 73.32128) (width 0.2) (layer "F.Cu") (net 12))
 (segment (start 131.14715 49.26075) (end 154.552876 49.26075) (width 0.2) (layer "F.Cu") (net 12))
 (segment (start 154.552876 49.26075) (end 155.22825 48.585376) (width 0.2) (layer "F.Cu") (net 12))
 (segment (start 155.22825 46.51812) (end 153.95388 45.24375) (width 0.2) (layer "F.Cu") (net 12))
 (segment (start 121.498436 94.111) (end 119.60775 92.220314) (width 0.2) (layer "F.Cu") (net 12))
 (segment (start 122.659064 94.111) (end 121.498436 94.111) (width 0.2) (layer "F.Cu") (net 12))
 (segment (start 122.00975 73.32128) (end 122.458434 73.32128) (width 0.2) (layer "F.Cu") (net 12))
 (segment (start 126.62675 53.78115) (end 131.14715 49.26075) (width 0.2) (layer "F.Cu") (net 12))
 (segment (start 126.62675 69.152964) (end 126.62675 53.78115) (width 0.2) (layer "F.Cu") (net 12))
 (segment (start 119.60775 73.32128) (end 120.31128 72.61775) (width 0.2) (layer "F.Cu") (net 12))
 (segment (start 143.51 92.71) (end 124.060064 92.71) (width 0.2) (layer "F.Cu") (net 12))
 (segment (start 124.060064 92.71) (end 122.659064 94.111) (width 0.2) (layer "F.Cu") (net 12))
 (segment (start 121.30622 72.61775) (end 122.00975 73.32128) (width 0.2) (layer "F.Cu") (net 12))
 (segment (start 155.22825 48.585376) (end 155.22825 46.51812) (width 0.2) (layer "F.Cu") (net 12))
 (segment (start 123.825 69.5325) (end 123.825 47.625) (width 0.2) (layer "F.Cu") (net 4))
 (segment (start 126.20625 47.625) (end 126.365 47.78375) (width 0.2) (layer "F.Cu") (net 4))
 (segment (start 123.825 47.625) (end 126.20625 47.625) (width 0.2) (layer "F.Cu") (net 4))
 (segment (start 126.365 47.78375) (end 136.80125 47.78375) (width 0.2) (layer "F.Cu") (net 4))
 (segment (start 122.07875 71.27875) (end 123.825 69.5325) (width 0.2) (layer "F.Cu") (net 4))
 (segment (start 142.875 59.53125) (end 130.96875 59.53125) (width 0.2) (layer "F.Cu") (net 5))
 (segment (start 142.875 69.13975) (end 142.875 69.33875) (width 0.2) (layer "F.Cu") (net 5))
 (segment (start 130.96875 59.53125) (end 130.96875 50.00625) (width 0.2) (layer "F.Cu") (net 5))
 (segment (start 130.96875 50.00625) (end 133.35 50.00625) (width 0.2) (layer "F.Cu") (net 5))
 (segment (start 133.6675 50.32375) (end 137.63625 50.32375) (width 0.2) (layer "F.Cu") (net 5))
 (segment (start 133.35 50.00625) (end 133.6675 50.32375) (width 0.2) (layer "F.Cu") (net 5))
 (segment (start 142.875 71.4375) (end 142.875 69.13975) (width 0.2) (layer "F.Cu") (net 5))
 (via (at 142.875 69.33875) (size 0.6) (drill 0.3) (layers "F.Cu" "B.Cu") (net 5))
 (via (at 142.875 59.53125) (size 0.6) (drill 0.3) (layers "F.Cu" "B.Cu") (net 5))
 (segment (start 142.875 69.33875) (end 142.875 59.53125) (width 0.2) (layer "B.Cu") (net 5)))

